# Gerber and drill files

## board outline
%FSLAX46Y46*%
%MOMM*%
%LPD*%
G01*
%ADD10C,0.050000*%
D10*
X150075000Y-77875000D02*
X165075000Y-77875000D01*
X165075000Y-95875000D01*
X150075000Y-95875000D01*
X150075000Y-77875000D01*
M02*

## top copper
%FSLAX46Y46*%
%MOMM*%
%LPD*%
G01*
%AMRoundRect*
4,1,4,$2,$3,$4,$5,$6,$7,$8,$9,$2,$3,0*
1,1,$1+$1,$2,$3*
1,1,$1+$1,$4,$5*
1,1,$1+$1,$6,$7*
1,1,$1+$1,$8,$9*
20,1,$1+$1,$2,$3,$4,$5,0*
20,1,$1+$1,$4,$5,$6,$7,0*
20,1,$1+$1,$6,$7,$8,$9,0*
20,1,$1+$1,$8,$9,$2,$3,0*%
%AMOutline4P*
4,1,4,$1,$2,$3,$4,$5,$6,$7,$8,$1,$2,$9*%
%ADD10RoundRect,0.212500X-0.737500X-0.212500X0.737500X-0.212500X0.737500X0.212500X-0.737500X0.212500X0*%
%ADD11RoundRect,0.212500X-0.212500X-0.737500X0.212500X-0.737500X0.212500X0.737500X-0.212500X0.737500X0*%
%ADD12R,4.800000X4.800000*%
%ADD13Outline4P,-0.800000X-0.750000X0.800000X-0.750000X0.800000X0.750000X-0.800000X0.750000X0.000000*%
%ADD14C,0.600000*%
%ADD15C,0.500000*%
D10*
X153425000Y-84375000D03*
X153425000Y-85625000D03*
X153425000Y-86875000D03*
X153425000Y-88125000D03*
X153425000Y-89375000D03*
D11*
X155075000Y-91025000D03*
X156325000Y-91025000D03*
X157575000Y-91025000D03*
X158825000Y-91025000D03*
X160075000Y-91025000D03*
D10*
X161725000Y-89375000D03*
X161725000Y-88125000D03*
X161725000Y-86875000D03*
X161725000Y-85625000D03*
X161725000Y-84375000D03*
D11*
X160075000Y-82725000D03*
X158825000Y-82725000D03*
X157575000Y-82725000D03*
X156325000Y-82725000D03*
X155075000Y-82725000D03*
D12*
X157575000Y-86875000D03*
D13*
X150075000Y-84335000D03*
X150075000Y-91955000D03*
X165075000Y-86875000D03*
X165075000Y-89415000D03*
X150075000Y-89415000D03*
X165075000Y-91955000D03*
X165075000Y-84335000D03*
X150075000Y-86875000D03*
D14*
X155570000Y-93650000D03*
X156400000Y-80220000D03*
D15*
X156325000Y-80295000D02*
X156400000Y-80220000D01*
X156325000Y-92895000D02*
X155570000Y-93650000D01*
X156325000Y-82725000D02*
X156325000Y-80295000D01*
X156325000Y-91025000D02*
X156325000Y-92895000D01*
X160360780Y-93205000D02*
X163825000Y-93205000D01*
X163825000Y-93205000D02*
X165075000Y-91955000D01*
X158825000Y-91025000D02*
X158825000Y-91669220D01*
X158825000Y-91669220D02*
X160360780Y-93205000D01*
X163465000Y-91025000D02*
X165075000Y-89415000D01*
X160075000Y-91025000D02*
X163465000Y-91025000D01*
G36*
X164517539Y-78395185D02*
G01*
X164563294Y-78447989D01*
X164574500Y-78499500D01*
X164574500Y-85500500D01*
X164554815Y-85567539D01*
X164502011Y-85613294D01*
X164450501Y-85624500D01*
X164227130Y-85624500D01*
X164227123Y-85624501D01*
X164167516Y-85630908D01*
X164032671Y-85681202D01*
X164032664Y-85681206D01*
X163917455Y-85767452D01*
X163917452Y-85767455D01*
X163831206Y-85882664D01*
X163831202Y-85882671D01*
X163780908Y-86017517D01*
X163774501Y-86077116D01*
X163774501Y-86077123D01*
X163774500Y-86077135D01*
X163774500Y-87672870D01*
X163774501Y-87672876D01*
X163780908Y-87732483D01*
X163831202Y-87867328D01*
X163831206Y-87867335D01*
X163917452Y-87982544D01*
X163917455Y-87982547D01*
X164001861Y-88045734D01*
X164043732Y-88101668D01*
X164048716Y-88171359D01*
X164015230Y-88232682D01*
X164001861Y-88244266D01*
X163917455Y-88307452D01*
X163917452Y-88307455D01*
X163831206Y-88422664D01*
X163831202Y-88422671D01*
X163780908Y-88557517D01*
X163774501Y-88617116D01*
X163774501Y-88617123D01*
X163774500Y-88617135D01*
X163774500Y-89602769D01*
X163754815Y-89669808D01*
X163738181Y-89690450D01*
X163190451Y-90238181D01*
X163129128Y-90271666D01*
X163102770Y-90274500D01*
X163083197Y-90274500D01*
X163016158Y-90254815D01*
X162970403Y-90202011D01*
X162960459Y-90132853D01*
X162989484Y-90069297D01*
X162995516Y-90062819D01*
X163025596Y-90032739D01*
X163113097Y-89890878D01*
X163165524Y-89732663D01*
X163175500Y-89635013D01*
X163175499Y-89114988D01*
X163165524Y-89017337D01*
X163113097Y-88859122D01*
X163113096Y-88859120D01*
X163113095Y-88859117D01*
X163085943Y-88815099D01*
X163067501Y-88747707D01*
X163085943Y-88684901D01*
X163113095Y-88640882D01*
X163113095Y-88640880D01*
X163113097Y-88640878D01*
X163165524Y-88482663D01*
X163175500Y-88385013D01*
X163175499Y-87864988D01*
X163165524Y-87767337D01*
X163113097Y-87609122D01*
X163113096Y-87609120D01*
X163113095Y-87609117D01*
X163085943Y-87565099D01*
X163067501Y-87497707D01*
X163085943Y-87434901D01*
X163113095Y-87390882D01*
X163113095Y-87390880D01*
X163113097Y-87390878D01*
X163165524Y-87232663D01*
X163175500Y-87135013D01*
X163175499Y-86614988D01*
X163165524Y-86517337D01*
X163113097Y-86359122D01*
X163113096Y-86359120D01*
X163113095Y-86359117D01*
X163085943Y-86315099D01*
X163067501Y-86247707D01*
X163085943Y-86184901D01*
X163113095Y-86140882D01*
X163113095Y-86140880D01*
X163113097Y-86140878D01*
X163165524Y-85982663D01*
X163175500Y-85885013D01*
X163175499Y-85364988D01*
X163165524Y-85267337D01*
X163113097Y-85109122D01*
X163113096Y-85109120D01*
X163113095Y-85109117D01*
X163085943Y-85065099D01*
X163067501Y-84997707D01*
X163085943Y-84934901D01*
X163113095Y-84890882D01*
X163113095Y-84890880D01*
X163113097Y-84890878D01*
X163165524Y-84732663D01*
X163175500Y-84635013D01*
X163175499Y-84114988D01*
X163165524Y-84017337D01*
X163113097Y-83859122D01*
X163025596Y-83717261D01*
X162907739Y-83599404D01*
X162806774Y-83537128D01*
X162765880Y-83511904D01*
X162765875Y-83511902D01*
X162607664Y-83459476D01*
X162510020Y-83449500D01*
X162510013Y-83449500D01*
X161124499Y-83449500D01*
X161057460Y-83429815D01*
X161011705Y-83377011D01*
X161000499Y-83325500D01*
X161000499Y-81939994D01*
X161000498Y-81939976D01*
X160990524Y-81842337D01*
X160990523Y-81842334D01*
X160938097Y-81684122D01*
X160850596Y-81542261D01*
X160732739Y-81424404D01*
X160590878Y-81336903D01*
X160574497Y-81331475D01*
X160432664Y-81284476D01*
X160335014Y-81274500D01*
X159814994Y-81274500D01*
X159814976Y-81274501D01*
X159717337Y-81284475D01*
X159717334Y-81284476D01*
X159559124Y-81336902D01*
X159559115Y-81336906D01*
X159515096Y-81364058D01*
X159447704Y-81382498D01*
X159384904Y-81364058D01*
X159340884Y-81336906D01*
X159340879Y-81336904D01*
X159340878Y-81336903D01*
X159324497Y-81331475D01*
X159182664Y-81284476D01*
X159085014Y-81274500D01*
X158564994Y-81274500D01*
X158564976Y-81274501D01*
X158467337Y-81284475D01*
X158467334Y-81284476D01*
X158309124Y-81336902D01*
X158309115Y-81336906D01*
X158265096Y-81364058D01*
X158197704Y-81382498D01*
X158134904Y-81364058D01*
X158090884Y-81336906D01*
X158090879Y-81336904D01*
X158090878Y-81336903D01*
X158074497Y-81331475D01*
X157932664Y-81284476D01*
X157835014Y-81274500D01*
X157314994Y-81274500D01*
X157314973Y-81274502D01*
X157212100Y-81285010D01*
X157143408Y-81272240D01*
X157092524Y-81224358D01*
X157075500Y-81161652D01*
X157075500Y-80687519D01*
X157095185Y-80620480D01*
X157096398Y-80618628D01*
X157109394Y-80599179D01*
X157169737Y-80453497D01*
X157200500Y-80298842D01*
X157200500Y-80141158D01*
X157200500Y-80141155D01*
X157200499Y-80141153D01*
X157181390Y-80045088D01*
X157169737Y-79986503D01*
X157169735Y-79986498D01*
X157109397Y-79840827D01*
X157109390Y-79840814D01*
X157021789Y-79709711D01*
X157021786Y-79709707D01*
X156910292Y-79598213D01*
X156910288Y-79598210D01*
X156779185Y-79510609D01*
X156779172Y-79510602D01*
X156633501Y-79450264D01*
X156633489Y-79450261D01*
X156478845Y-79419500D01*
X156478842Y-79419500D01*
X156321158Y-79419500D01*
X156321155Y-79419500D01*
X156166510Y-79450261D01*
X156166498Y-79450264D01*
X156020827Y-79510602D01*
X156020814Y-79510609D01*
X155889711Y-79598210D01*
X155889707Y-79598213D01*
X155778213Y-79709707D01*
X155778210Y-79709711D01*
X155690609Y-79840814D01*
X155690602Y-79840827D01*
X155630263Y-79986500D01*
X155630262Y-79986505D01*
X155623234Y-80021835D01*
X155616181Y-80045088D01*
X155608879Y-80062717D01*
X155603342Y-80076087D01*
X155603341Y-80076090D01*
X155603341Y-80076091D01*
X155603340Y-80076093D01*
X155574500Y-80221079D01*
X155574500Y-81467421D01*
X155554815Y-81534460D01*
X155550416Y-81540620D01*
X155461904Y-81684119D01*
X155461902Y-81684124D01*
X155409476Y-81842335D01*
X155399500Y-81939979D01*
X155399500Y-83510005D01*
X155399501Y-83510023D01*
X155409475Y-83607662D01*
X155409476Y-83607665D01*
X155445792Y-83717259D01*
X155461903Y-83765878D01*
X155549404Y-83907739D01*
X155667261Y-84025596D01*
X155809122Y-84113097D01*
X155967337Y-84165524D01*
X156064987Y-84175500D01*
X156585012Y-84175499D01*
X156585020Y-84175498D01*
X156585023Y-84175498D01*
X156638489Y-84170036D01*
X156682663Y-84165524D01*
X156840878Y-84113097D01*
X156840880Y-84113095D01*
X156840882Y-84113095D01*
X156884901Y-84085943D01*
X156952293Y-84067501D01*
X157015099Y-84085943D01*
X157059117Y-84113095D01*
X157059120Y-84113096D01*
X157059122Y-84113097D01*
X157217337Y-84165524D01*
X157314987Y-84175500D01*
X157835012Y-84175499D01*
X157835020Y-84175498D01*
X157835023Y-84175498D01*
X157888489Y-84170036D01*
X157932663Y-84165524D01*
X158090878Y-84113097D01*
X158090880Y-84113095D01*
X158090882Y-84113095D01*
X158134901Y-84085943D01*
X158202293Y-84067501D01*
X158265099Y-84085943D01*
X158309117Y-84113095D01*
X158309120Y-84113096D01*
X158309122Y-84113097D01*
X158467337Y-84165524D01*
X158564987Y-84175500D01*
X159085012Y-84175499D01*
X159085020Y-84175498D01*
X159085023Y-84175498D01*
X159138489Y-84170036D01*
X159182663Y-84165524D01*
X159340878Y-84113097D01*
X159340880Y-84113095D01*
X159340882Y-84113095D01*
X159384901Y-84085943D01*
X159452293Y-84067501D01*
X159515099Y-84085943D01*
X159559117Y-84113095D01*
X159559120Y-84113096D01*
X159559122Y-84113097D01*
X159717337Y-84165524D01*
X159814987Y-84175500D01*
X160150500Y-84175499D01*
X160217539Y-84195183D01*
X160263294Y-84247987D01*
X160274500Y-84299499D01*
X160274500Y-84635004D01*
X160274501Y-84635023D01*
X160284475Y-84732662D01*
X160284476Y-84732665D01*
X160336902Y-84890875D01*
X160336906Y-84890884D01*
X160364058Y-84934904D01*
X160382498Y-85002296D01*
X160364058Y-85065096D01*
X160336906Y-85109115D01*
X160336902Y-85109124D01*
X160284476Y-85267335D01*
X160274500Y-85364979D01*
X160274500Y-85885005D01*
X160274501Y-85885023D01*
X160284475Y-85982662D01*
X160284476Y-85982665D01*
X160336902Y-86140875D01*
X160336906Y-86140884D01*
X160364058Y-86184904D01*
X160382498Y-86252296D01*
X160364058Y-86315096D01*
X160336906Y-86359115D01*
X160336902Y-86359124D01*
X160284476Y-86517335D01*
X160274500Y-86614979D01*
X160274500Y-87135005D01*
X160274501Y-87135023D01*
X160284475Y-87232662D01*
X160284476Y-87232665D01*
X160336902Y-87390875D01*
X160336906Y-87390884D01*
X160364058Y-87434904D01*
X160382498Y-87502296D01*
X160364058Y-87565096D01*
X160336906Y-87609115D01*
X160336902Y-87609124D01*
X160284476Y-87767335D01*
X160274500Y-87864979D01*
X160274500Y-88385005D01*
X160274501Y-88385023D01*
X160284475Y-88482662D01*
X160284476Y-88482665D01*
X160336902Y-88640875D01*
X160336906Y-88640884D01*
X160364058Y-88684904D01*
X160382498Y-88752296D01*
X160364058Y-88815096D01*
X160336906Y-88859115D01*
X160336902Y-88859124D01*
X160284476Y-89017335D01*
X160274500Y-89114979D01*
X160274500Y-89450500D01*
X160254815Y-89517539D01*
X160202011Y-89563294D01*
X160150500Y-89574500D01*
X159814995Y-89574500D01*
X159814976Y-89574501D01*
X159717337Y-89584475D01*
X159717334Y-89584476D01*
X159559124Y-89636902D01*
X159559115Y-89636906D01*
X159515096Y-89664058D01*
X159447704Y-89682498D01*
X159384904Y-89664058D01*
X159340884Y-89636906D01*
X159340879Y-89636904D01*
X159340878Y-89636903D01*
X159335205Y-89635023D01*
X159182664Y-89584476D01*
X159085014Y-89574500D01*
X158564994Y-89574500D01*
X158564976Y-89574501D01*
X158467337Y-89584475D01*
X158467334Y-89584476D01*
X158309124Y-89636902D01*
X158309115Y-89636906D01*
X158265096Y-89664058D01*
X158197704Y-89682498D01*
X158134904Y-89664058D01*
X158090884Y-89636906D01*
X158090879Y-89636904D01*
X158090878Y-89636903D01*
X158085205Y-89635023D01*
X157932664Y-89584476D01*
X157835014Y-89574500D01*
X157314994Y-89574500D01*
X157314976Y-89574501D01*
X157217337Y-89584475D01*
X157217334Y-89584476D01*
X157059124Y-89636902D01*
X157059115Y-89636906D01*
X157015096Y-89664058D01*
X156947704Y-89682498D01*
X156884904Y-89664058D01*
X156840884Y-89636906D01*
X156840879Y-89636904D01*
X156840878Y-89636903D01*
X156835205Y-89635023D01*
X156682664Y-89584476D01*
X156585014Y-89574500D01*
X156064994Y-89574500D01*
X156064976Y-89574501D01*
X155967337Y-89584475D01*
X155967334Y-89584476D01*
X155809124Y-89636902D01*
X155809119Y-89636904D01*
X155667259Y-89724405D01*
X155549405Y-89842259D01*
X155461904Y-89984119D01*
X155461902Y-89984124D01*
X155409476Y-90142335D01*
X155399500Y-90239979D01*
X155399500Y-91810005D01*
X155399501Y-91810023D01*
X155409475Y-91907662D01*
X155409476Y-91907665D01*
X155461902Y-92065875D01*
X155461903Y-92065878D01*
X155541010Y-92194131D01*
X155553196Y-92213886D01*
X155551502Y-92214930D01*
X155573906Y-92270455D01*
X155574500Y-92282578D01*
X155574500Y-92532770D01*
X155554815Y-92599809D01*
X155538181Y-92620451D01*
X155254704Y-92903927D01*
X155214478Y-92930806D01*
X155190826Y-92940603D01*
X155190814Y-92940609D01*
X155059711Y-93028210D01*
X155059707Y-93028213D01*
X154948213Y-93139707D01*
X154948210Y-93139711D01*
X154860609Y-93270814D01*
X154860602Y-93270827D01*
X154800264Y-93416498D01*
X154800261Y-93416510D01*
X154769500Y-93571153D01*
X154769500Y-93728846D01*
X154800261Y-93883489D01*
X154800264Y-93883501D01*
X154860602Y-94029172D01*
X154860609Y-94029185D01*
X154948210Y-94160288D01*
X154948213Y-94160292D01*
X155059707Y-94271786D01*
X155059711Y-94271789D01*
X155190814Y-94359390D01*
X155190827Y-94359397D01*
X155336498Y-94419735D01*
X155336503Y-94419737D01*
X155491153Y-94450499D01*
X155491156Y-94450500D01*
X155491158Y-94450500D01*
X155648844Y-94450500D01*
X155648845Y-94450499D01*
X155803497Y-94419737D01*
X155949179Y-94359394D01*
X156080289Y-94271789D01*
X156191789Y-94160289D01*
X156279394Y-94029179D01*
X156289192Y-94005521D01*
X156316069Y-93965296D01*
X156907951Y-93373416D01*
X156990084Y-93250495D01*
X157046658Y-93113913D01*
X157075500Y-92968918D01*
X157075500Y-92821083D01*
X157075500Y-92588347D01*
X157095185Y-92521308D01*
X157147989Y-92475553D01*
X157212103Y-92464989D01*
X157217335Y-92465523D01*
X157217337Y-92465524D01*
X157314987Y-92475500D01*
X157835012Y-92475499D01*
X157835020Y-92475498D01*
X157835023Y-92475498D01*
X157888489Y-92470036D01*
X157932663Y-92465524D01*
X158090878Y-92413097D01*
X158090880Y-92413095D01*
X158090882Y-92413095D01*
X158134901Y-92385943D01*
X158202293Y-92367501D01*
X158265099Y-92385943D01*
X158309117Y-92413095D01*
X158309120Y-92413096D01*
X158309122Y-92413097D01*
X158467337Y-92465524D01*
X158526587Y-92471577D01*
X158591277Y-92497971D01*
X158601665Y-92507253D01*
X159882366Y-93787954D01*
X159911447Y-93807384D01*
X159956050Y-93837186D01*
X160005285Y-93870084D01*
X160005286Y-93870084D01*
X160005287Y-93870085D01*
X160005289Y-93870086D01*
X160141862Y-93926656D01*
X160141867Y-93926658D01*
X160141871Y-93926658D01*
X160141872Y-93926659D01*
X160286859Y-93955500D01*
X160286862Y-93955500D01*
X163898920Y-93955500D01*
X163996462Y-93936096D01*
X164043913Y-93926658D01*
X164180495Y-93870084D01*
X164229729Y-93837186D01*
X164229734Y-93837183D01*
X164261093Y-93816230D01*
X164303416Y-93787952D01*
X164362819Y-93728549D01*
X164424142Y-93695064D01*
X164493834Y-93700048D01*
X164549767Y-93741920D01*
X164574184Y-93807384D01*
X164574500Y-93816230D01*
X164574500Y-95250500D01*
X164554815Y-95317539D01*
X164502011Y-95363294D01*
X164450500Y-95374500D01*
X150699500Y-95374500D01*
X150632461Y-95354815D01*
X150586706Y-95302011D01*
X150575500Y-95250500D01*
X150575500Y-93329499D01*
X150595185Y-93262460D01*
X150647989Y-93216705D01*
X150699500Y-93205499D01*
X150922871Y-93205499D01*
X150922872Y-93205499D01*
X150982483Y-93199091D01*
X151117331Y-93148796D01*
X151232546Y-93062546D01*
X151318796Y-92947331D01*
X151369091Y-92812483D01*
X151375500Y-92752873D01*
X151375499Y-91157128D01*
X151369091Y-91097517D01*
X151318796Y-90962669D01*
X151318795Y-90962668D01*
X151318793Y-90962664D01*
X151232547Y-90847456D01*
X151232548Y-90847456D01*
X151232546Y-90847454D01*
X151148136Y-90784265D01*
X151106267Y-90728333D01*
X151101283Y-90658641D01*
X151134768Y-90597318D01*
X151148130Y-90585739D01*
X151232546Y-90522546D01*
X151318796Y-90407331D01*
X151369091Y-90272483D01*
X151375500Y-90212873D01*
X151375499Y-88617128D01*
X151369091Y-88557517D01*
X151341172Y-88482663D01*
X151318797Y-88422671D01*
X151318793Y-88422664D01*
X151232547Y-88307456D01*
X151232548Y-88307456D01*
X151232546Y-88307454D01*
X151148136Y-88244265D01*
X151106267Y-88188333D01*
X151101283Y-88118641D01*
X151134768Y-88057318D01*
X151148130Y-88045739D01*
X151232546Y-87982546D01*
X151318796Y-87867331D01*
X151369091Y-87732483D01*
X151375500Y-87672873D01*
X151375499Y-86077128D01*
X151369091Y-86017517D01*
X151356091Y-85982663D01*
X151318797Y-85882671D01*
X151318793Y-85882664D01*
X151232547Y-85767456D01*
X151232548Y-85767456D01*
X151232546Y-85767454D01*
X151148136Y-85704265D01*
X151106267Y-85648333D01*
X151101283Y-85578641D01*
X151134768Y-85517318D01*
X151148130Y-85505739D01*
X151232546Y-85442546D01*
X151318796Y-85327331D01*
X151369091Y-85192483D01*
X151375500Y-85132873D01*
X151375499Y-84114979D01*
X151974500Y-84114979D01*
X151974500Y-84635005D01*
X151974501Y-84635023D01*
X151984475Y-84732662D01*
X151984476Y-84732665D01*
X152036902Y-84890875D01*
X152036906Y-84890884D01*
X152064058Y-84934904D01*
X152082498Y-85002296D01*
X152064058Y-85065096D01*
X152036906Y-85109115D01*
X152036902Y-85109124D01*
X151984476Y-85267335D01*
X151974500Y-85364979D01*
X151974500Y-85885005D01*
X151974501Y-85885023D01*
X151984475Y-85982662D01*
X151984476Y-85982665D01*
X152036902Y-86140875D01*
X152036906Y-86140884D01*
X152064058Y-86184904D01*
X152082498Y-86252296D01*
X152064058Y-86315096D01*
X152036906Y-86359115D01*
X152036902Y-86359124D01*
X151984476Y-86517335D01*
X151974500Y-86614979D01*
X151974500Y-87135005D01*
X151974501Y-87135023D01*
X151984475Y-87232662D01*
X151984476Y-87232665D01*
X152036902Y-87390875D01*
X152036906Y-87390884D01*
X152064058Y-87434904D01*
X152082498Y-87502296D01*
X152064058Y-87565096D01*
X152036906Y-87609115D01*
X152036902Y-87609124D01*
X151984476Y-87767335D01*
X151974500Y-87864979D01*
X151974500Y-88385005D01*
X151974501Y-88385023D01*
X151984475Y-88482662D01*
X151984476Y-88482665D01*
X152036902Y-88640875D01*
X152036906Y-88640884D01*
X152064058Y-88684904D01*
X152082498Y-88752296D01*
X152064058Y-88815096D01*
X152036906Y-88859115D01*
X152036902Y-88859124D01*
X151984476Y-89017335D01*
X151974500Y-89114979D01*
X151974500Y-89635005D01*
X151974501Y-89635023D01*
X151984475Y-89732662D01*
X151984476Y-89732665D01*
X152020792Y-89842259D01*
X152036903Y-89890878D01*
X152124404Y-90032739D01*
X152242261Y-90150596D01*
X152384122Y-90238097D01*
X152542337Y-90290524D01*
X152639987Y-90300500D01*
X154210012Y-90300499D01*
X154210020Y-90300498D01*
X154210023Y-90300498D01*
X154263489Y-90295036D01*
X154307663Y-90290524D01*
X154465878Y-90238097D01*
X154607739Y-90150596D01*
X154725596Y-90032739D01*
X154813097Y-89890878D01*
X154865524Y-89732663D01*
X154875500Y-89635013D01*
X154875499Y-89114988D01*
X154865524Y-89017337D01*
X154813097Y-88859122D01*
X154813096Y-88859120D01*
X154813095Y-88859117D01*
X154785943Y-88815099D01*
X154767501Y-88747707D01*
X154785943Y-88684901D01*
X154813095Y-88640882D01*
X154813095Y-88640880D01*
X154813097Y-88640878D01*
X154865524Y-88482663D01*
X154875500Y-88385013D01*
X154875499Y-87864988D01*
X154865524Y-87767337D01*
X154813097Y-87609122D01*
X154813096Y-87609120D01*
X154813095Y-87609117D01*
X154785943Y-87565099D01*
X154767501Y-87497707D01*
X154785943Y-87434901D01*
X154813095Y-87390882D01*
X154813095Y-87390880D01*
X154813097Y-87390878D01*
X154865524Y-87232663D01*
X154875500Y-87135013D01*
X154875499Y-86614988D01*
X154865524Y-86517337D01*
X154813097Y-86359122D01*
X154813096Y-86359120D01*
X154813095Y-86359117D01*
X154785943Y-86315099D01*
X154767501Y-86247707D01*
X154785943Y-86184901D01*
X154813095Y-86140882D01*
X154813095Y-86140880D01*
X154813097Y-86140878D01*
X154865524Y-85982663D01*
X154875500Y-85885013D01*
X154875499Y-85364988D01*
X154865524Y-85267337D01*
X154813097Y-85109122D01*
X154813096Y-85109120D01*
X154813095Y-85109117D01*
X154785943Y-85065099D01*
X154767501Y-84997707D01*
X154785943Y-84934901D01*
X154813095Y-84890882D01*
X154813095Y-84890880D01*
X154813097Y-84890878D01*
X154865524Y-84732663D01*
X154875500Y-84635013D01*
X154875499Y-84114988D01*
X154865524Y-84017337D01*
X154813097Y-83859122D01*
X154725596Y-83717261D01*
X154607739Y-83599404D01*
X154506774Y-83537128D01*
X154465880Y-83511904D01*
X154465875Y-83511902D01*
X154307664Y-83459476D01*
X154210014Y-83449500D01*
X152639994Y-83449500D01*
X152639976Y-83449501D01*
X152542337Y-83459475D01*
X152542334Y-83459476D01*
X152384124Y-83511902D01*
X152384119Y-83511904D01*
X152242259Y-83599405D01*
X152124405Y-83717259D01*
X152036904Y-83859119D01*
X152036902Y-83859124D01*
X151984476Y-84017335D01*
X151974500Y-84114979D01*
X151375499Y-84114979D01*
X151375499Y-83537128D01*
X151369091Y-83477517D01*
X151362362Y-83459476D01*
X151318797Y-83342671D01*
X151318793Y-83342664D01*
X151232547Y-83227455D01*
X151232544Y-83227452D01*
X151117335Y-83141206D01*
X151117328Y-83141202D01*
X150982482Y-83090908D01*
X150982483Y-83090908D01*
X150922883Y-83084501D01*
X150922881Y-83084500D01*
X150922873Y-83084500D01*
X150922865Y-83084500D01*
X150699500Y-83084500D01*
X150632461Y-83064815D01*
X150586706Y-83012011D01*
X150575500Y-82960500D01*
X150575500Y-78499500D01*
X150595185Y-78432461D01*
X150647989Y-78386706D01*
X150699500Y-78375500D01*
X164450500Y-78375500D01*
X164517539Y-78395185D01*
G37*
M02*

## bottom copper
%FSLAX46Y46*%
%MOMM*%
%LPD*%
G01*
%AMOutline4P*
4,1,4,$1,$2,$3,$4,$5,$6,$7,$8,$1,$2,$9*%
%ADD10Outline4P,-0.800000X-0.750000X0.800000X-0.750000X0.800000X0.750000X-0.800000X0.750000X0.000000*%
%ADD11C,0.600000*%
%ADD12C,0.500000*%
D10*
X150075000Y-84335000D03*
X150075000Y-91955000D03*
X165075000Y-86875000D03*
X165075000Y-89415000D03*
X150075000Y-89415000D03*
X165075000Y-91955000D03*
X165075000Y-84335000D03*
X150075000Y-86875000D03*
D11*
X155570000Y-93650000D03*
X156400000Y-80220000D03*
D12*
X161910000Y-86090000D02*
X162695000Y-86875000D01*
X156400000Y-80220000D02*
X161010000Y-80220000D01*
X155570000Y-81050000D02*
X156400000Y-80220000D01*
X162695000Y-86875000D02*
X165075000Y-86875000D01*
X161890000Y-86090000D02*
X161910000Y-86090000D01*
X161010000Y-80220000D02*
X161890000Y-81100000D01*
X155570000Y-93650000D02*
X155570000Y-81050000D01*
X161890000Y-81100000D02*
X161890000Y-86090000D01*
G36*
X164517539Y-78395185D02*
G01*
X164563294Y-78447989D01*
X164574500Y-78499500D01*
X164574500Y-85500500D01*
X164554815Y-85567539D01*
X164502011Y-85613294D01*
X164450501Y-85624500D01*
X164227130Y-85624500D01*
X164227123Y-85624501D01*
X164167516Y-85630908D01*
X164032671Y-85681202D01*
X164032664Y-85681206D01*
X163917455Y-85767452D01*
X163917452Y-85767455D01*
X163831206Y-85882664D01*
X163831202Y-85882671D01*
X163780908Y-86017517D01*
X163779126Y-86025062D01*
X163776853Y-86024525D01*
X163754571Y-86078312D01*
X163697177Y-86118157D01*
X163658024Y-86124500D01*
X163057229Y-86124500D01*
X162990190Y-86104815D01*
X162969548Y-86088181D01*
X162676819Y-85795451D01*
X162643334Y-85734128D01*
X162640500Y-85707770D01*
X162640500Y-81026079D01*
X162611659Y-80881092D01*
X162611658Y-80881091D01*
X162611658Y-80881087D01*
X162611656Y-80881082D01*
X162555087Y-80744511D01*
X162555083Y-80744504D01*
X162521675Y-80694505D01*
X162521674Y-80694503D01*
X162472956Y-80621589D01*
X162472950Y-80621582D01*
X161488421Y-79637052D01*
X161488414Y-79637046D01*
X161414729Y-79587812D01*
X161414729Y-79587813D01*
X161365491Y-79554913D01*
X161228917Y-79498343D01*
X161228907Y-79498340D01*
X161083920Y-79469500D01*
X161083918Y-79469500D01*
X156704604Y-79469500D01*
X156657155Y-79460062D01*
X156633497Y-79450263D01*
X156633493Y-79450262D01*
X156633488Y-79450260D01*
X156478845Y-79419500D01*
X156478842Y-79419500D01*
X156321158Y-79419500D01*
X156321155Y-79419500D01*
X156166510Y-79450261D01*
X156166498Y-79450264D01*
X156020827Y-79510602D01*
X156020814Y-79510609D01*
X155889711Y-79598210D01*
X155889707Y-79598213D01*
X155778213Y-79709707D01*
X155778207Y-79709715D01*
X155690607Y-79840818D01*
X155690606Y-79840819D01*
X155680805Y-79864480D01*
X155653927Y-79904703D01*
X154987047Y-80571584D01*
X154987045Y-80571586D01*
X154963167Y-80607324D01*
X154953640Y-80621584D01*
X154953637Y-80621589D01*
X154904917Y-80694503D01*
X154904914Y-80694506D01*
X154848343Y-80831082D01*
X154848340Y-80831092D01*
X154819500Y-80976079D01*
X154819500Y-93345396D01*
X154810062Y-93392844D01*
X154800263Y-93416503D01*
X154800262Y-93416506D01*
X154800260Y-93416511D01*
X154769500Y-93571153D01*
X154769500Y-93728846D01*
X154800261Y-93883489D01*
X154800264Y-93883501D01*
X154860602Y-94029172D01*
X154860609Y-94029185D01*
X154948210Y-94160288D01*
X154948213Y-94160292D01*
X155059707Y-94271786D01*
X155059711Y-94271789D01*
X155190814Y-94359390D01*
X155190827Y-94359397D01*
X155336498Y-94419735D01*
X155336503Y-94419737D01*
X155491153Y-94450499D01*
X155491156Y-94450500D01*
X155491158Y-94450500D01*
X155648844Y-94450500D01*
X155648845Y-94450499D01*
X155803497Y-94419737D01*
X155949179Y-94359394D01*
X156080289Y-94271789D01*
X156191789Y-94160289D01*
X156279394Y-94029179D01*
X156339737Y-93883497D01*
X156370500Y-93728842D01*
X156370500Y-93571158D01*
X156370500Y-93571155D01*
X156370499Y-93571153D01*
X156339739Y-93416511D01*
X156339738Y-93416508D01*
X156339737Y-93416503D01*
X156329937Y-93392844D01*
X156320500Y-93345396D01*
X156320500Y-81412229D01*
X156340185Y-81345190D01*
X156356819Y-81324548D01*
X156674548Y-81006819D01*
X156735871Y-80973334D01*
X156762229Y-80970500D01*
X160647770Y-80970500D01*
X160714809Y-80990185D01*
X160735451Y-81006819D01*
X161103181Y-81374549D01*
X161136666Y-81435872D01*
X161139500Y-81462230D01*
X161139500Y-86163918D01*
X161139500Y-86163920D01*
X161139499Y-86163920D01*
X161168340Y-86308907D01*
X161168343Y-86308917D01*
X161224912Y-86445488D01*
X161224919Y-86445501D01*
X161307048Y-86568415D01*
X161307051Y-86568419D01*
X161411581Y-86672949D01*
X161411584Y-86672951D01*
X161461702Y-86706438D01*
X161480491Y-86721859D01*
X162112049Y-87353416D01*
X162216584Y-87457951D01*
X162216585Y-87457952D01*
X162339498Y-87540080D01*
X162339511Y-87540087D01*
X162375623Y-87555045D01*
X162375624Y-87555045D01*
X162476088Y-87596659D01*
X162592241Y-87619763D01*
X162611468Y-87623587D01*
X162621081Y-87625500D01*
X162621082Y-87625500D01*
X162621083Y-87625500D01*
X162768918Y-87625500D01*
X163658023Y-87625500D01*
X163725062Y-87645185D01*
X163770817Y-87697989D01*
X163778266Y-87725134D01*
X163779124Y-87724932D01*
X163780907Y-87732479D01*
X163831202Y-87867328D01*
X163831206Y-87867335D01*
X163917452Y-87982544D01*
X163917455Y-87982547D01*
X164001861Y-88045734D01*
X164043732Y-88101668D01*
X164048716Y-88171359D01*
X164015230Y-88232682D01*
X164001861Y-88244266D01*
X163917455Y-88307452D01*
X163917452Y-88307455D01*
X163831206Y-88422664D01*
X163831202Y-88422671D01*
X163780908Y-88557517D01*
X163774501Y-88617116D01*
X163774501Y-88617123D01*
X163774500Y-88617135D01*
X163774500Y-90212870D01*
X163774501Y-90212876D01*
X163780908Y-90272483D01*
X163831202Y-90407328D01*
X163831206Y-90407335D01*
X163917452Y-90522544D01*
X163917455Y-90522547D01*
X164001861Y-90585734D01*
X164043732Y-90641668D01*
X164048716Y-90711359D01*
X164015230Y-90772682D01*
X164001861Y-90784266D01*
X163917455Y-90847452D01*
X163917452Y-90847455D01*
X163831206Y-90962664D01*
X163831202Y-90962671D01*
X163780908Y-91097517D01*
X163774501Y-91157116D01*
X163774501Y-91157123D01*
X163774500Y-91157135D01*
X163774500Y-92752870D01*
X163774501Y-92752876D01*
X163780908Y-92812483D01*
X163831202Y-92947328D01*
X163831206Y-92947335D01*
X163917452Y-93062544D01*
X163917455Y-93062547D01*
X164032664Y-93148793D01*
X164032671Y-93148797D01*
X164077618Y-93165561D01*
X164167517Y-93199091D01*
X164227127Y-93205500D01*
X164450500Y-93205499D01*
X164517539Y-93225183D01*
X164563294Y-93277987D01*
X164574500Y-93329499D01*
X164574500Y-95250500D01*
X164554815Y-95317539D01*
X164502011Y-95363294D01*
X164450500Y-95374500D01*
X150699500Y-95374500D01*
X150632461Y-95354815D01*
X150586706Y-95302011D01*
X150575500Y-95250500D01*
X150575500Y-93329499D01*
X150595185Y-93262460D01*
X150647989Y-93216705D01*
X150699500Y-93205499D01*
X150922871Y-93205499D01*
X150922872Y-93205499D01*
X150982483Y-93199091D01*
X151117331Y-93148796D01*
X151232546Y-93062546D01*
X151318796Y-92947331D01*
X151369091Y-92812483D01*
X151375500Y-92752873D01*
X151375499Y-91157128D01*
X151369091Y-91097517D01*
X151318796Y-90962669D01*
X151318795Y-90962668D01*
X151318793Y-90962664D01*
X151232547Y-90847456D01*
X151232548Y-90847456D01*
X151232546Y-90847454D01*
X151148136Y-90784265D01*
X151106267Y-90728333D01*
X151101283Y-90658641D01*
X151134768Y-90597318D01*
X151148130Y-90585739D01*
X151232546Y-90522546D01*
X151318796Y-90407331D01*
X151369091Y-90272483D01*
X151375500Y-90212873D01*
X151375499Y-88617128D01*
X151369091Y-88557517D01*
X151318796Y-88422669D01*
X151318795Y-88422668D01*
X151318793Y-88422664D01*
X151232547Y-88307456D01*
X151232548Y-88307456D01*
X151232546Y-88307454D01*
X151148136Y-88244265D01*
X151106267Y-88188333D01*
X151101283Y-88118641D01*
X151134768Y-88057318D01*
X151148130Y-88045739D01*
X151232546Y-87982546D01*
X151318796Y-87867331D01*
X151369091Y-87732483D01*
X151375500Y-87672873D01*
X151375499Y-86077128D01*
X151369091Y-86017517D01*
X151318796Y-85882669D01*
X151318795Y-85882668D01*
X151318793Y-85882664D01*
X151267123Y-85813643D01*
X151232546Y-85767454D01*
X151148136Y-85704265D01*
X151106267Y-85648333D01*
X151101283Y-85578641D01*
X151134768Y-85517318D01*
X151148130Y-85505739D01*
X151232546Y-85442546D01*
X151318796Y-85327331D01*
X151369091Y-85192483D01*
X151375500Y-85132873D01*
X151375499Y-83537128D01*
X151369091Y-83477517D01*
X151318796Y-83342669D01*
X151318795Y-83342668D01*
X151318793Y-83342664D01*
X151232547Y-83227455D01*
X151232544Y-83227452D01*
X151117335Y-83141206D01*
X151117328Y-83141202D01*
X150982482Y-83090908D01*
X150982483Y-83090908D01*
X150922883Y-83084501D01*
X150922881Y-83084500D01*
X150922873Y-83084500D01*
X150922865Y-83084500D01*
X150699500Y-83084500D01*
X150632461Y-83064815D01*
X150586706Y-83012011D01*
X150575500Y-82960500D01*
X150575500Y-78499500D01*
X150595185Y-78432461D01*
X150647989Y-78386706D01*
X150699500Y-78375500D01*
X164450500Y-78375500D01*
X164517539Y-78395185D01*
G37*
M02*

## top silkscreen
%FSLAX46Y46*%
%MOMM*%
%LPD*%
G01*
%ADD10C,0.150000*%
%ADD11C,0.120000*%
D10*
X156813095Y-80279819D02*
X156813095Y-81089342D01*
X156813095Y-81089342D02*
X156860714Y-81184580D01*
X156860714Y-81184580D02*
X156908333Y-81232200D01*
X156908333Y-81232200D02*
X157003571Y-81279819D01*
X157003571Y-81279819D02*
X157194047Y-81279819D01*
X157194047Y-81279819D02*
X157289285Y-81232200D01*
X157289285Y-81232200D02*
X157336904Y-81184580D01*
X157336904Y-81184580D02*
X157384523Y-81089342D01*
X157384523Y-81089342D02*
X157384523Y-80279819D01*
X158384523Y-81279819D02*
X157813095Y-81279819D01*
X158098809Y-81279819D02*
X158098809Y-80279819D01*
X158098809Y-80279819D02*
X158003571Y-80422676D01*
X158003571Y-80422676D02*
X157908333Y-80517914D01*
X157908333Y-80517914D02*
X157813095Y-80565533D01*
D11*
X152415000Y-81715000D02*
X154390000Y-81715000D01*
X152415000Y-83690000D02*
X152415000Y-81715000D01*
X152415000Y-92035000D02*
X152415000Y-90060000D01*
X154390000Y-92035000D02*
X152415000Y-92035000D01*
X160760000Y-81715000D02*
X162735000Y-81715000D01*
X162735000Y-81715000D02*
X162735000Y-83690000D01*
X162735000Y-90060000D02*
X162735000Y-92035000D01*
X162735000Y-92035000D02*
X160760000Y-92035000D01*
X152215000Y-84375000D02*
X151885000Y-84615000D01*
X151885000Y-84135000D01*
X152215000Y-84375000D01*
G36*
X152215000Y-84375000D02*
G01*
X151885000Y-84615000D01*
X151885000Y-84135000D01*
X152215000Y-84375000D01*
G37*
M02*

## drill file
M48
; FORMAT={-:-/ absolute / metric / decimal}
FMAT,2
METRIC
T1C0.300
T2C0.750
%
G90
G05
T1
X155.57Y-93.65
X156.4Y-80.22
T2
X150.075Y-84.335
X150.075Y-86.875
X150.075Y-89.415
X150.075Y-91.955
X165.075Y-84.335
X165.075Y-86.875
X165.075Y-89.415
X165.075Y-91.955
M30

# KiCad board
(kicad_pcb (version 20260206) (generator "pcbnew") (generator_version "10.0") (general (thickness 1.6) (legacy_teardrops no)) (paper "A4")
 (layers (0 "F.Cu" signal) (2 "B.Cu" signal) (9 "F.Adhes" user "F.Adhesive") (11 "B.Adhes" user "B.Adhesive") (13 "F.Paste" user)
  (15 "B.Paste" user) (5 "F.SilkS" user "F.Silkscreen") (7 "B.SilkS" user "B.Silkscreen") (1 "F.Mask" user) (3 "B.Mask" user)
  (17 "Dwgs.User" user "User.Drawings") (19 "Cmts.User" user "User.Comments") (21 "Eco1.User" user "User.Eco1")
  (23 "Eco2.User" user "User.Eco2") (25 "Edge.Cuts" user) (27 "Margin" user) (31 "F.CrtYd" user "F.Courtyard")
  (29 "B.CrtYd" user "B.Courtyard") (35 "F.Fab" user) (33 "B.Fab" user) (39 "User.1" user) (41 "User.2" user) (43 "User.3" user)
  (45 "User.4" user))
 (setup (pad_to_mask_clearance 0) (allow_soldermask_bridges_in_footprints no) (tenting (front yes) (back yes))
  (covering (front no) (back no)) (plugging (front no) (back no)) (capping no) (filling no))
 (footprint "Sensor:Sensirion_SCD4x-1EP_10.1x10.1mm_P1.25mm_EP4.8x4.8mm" (layer "F.Cu") (at 157.575 86.875)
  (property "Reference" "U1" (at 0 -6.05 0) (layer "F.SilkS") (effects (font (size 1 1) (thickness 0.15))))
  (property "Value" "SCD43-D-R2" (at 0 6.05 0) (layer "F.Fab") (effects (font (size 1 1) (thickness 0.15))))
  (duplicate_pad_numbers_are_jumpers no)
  (fp_line (start -5.16 -5.16) (end -3.185 -5.16) (stroke (width 0.12) (type solid)) (layer "F.SilkS"))
  (fp_line (start -5.16 -3.185) (end -5.16 -5.16) (stroke (width 0.12) (type solid)) (layer "F.SilkS"))
  (fp_line (start -5.16 5.16) (end -5.16 3.185) (stroke (width 0.12) (type solid)) (layer "F.SilkS"))
  (fp_line (start -3.185 5.16) (end -5.16 5.16) (stroke (width 0.12) (type solid)) (layer "F.SilkS"))
  (fp_line (start 3.185 -5.16) (end 5.16 -5.16) (stroke (width 0.12) (type solid)) (layer "F.SilkS"))
  (fp_line (start 5.16 -5.16) (end 5.16 -3.185) (stroke (width 0.12) (type solid)) (layer "F.SilkS"))
  (fp_line (start 5.16 3.185) (end 5.16 5.16) (stroke (width 0.12) (type solid)) (layer "F.SilkS"))
  (fp_line (start 5.16 5.16) (end 3.185 5.16) (stroke (width 0.12) (type solid)) (layer "F.SilkS"))
  (fp_poly (pts (xy -5.36 -2.5) (xy -5.69 -2.26) (xy -5.69 -2.74)) (stroke (width 0.12) (type solid)) (fill yes) (layer "F.SilkS"))
  (pad "" smd roundrect (at -1.2 -1.2) (size 1.93 1.93) (layers "F.Paste") (roundrect_rratio 0.129534))
  (pad "" smd roundrect (at -1.2 1.2) (size 1.93 1.93) (layers "F.Paste") (roundrect_rratio 0.129534))
  (pad "" smd roundrect (at 1.2 -1.2) (size 1.93 1.93) (layers "F.Paste") (roundrect_rratio 0.129534))
  (pad "" smd roundrect (at 1.2 1.2) (size 1.93 1.93) (layers "F.Paste") (roundrect_rratio 0.129534))
  (pad "1" smd roundrect (at -4.15 -2.5) (size 1.9 0.85) (layers "F.Cu" "F.Mask" "F.Paste") (roundrect_rratio 0.25))
  (pad "2" smd roundrect (at -4.15 -1.25) (size 1.9 0.85) (layers "F.Cu" "F.Mask" "F.Paste") (roundrect_rratio 0.25))
  (pad "3" smd roundrect (at -4.15 0) (size 1.9 0.85) (layers "F.Cu" "F.Mask" "F.Paste") (roundrect_rratio 0.25))
  (pad "4" smd roundrect (at -4.15 1.25) (size 1.9 0.85) (layers "F.Cu" "F.Mask" "F.Paste") (roundrect_rratio 0.25))
  (pad "5" smd roundrect (at -4.15 2.5) (size 1.9 0.85) (layers "F.Cu" "F.Mask" "F.Paste") (roundrect_rratio 0.25))
  (pad "6" smd roundrect (at -2.5 4.15) (size 0.85 1.9) (layers "F.Cu" "F.Mask" "F.Paste") (roundrect_rratio 0.25) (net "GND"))
  (pad "7" smd roundrect (at -1.25 4.15) (size 0.85 1.9) (layers "F.Cu" "F.Mask" "F.Paste") (roundrect_rratio 0.25) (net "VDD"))
  (pad "8" smd roundrect (at 0 4.15) (size 0.85 1.9) (layers "F.Cu" "F.Mask" "F.Paste") (roundrect_rratio 0.25))
  (pad "9" smd roundrect (at 1.25 4.15) (size 0.85 1.9) (layers "F.Cu" "F.Mask" "F.Paste") (roundrect_rratio 0.25) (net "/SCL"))
  (pad "10" smd roundrect (at 2.5 4.15) (size 0.85 1.9) (layers "F.Cu" "F.Mask" "F.Paste") (roundrect_rratio 0.25) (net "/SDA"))
  (pad "11" smd roundrect (at 4.15 2.5) (size 1.9 0.85) (layers "F.Cu" "F.Mask" "F.Paste") (roundrect_rratio 0.25))
  (pad "12" smd roundrect (at 4.15 1.25) (size 1.9 0.85) (layers "F.Cu" "F.Mask" "F.Paste") (roundrect_rratio 0.25))
  (pad "13" smd roundrect (at 4.15 0) (size 1.9 0.85) (layers "F.Cu" "F.Mask" "F.Paste") (roundrect_rratio 0.25))
  (pad "14" smd roundrect (at 4.15 -1.25) (size 1.9 0.85) (layers "F.Cu" "F.Mask" "F.Paste") (roundrect_rratio 0.25))
  (pad "15" smd roundrect (at 4.15 -2.5) (size 1.9 0.85) (layers "F.Cu" "F.Mask" "F.Paste") (roundrect_rratio 0.25))
  (pad "16" smd roundrect (at 2.5 -4.15) (size 0.85 1.9) (layers "F.Cu" "F.Mask" "F.Paste") (roundrect_rratio 0.25))
  (pad "17" smd roundrect (at 1.25 -4.15) (size 0.85 1.9) (layers "F.Cu" "F.Mask" "F.Paste") (roundrect_rratio 0.25))
  (pad "18" smd roundrect (at 0 -4.15) (size 0.85 1.9) (layers "F.Cu" "F.Mask" "F.Paste") (roundrect_rratio 0.25))
  (pad "19" smd roundrect (at -1.25 -4.15) (size 0.85 1.9) (layers "F.Cu" "F.Mask" "F.Paste") (roundrect_rratio 0.25) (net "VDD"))
  (pad "20" smd roundrect (at -2.5 -4.15) (size 0.85 1.9) (layers "F.Cu" "F.Mask" "F.Paste") (roundrect_rratio 0.25) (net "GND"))
  (pad "21" smd rect (at 0 0) (size 4.8 4.8) (layers "F.Cu" "F.Mask") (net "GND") (zone_connect 2)))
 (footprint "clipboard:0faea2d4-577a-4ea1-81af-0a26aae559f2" (layer "F.Cu") (at 150.075 84.335)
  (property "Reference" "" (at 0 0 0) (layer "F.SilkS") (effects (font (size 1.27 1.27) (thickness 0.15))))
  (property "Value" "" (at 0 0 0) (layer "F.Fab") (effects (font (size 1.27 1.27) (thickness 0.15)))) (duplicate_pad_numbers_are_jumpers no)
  (pad "1" thru_hole trapezoid (at 0 0) (size 1.6 1.5) (drill 0.75) (layers "*.Cu" "*.Mask") (remove_unused_layers no)))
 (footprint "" (layer "F.Cu") (at 150.075 91.955)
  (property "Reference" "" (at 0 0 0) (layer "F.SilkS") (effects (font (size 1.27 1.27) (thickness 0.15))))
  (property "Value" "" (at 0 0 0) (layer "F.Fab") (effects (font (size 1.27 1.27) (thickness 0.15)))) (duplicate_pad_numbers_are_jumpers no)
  (pad "1" thru_hole trapezoid (at 0 0) (size 1.6 1.5) (drill 0.75) (layers "*.Cu" "*.Mask") (remove_unused_layers no)))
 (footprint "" (layer "F.Cu") (at 165.075 86.875)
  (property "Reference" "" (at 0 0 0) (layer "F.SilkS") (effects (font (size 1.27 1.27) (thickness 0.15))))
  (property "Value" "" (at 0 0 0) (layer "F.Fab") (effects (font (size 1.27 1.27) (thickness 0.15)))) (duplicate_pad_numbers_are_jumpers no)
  (pad "1" thru_hole trapezoid (at 0 0) (size 1.6 1.5) (drill 0.75) (layers "*.Cu" "*.Mask") (remove_unused_layers no) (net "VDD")))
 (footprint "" (layer "F.Cu") (at 165.075 89.415)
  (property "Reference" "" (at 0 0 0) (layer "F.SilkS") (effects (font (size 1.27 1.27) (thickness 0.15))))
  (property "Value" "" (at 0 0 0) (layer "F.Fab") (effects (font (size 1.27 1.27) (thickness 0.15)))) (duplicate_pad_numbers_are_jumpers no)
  (pad "1" thru_hole trapezoid (at 0 0) (size 1.6 1.5) (drill 0.75) (layers "*.Cu" "*.Mask") (remove_unused_layers no) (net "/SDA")))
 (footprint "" (layer "F.Cu") (at 150.075 89.415)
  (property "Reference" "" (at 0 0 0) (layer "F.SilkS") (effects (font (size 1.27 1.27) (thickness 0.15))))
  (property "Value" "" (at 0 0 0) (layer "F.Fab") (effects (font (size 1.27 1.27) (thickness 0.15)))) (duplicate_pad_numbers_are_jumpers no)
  (pad "1" thru_hole trapezoid (at 0 0) (size 1.6 1.5) (drill 0.75) (layers "*.Cu" "*.Mask") (remove_unused_layers no)))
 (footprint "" (layer "F.Cu") (at 165.075 91.955)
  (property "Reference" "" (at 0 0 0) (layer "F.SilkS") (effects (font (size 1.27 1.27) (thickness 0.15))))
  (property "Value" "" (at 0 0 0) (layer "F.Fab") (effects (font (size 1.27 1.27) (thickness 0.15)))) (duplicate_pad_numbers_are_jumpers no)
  (pad "1" thru_hole trapezoid (at 0 0) (size 1.6 1.5) (drill 0.75) (layers "*.Cu" "*.Mask") (remove_unused_layers no) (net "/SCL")))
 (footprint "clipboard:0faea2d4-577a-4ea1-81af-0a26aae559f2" (layer "F.Cu") (at 165.075 84.335)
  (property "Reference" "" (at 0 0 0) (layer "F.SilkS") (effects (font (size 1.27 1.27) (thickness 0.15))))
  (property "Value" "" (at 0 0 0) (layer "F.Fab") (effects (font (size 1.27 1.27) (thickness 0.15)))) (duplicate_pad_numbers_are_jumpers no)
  (pad "1" thru_hole trapezoid (at 0 0) (size 1.6 1.5) (drill 0.75) (layers "*.Cu" "*.Mask") (remove_unused_layers no) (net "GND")))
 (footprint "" (layer "F.Cu") (at 150.075 86.875)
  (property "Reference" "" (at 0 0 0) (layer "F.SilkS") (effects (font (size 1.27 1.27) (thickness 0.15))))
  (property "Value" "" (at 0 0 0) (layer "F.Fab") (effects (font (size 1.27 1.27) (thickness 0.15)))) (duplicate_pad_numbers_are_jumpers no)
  (pad "1" thru_hole trapezoid (at 0 0) (size 1.6 1.5) (drill 0.75) (layers "*.Cu" "*.Mask") (remove_unused_layers no)))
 (gr_rect (start 150.075 77.875) (end 165.075 95.875) (stroke (width 0.05) (type solid)) (fill no) (layer "Edge.Cuts"))
 (segment (start 156.325 80.295) (end 156.4 80.22) (width 0.5) (layer "F.Cu") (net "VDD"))
 (segment (start 156.325 92.895) (end 155.57 93.65) (width 0.5) (layer "F.Cu") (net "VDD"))
 (segment (start 156.325 82.725) (end 156.325 80.295) (width 0.5) (layer "F.Cu") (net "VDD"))
 (segment (start 156.325 91.025) (end 156.325 92.895) (width 0.5) (layer "F.Cu") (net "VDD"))
 (via (at 155.57 93.65) (size 0.6) (drill 0.3) (layers "F.Cu" "B.Cu") (capping no) (covering (front no) (back no))
  (plugging (front no) (back no)) (filling no) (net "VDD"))
 (via (at 156.4 80.22) (size 0.6) (drill 0.3) (layers "F.Cu" "B.Cu") (capping no) (covering (front no) (back no))
  (plugging (front no) (back no)) (filling no) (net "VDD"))
 (segment (start 161.91 86.09) (end 162.695 86.875) (width 0.5) (layer "B.Cu") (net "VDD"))
 (segment (start 156.4 80.22) (end 161.01 80.22) (width 0.5) (layer "B.Cu") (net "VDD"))
 (segment (start 155.57 81.05) (end 156.4 80.22) (width 0.5) (layer "B.Cu") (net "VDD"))
 (segment (start 162.695 86.875) (end 165.075 86.875) (width 0.5) (layer "B.Cu") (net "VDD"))
 (segment (start 161.89 86.09) (end 161.91 86.09) (width 0.5) (layer "B.Cu") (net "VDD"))
 (segment (start 161.01 80.22) (end 161.89 81.1) (width 0.5) (layer "B.Cu") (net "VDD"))
 (segment (start 155.57 93.65) (end 155.57 81.05) (width 0.5) (layer "B.Cu") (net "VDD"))
 (segment (start 161.89 81.1) (end 161.89 86.09) (width 0.5) (layer "B.Cu") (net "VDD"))
 (segment (start 160.36078 93.205) (end 163.825 93.205) (width 0.5) (layer "F.Cu") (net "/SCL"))
 (segment (start 163.825 93.205) (end 165.075 91.955) (width 0.5) (layer "F.Cu") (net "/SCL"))
 (segment (start 158.825 91.025) (end 158.825 91.66922) (width 0.5) (layer "F.Cu") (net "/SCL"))
 (segment (start 158.825 91.66922) (end 160.36078 93.205) (width 0.5) (layer "F.Cu") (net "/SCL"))
 (segment (start 163.465 91.025) (end 165.075 89.415) (width 0.5) (layer "F.Cu") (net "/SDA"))
 (segment (start 160.075 91.025) (end 163.465 91.025) (width 0.5) (layer "F.Cu") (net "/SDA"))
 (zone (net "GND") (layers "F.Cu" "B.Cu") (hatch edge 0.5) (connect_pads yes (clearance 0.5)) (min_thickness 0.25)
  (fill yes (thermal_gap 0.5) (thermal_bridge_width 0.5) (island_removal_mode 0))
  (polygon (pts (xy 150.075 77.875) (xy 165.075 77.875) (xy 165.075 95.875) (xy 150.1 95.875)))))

